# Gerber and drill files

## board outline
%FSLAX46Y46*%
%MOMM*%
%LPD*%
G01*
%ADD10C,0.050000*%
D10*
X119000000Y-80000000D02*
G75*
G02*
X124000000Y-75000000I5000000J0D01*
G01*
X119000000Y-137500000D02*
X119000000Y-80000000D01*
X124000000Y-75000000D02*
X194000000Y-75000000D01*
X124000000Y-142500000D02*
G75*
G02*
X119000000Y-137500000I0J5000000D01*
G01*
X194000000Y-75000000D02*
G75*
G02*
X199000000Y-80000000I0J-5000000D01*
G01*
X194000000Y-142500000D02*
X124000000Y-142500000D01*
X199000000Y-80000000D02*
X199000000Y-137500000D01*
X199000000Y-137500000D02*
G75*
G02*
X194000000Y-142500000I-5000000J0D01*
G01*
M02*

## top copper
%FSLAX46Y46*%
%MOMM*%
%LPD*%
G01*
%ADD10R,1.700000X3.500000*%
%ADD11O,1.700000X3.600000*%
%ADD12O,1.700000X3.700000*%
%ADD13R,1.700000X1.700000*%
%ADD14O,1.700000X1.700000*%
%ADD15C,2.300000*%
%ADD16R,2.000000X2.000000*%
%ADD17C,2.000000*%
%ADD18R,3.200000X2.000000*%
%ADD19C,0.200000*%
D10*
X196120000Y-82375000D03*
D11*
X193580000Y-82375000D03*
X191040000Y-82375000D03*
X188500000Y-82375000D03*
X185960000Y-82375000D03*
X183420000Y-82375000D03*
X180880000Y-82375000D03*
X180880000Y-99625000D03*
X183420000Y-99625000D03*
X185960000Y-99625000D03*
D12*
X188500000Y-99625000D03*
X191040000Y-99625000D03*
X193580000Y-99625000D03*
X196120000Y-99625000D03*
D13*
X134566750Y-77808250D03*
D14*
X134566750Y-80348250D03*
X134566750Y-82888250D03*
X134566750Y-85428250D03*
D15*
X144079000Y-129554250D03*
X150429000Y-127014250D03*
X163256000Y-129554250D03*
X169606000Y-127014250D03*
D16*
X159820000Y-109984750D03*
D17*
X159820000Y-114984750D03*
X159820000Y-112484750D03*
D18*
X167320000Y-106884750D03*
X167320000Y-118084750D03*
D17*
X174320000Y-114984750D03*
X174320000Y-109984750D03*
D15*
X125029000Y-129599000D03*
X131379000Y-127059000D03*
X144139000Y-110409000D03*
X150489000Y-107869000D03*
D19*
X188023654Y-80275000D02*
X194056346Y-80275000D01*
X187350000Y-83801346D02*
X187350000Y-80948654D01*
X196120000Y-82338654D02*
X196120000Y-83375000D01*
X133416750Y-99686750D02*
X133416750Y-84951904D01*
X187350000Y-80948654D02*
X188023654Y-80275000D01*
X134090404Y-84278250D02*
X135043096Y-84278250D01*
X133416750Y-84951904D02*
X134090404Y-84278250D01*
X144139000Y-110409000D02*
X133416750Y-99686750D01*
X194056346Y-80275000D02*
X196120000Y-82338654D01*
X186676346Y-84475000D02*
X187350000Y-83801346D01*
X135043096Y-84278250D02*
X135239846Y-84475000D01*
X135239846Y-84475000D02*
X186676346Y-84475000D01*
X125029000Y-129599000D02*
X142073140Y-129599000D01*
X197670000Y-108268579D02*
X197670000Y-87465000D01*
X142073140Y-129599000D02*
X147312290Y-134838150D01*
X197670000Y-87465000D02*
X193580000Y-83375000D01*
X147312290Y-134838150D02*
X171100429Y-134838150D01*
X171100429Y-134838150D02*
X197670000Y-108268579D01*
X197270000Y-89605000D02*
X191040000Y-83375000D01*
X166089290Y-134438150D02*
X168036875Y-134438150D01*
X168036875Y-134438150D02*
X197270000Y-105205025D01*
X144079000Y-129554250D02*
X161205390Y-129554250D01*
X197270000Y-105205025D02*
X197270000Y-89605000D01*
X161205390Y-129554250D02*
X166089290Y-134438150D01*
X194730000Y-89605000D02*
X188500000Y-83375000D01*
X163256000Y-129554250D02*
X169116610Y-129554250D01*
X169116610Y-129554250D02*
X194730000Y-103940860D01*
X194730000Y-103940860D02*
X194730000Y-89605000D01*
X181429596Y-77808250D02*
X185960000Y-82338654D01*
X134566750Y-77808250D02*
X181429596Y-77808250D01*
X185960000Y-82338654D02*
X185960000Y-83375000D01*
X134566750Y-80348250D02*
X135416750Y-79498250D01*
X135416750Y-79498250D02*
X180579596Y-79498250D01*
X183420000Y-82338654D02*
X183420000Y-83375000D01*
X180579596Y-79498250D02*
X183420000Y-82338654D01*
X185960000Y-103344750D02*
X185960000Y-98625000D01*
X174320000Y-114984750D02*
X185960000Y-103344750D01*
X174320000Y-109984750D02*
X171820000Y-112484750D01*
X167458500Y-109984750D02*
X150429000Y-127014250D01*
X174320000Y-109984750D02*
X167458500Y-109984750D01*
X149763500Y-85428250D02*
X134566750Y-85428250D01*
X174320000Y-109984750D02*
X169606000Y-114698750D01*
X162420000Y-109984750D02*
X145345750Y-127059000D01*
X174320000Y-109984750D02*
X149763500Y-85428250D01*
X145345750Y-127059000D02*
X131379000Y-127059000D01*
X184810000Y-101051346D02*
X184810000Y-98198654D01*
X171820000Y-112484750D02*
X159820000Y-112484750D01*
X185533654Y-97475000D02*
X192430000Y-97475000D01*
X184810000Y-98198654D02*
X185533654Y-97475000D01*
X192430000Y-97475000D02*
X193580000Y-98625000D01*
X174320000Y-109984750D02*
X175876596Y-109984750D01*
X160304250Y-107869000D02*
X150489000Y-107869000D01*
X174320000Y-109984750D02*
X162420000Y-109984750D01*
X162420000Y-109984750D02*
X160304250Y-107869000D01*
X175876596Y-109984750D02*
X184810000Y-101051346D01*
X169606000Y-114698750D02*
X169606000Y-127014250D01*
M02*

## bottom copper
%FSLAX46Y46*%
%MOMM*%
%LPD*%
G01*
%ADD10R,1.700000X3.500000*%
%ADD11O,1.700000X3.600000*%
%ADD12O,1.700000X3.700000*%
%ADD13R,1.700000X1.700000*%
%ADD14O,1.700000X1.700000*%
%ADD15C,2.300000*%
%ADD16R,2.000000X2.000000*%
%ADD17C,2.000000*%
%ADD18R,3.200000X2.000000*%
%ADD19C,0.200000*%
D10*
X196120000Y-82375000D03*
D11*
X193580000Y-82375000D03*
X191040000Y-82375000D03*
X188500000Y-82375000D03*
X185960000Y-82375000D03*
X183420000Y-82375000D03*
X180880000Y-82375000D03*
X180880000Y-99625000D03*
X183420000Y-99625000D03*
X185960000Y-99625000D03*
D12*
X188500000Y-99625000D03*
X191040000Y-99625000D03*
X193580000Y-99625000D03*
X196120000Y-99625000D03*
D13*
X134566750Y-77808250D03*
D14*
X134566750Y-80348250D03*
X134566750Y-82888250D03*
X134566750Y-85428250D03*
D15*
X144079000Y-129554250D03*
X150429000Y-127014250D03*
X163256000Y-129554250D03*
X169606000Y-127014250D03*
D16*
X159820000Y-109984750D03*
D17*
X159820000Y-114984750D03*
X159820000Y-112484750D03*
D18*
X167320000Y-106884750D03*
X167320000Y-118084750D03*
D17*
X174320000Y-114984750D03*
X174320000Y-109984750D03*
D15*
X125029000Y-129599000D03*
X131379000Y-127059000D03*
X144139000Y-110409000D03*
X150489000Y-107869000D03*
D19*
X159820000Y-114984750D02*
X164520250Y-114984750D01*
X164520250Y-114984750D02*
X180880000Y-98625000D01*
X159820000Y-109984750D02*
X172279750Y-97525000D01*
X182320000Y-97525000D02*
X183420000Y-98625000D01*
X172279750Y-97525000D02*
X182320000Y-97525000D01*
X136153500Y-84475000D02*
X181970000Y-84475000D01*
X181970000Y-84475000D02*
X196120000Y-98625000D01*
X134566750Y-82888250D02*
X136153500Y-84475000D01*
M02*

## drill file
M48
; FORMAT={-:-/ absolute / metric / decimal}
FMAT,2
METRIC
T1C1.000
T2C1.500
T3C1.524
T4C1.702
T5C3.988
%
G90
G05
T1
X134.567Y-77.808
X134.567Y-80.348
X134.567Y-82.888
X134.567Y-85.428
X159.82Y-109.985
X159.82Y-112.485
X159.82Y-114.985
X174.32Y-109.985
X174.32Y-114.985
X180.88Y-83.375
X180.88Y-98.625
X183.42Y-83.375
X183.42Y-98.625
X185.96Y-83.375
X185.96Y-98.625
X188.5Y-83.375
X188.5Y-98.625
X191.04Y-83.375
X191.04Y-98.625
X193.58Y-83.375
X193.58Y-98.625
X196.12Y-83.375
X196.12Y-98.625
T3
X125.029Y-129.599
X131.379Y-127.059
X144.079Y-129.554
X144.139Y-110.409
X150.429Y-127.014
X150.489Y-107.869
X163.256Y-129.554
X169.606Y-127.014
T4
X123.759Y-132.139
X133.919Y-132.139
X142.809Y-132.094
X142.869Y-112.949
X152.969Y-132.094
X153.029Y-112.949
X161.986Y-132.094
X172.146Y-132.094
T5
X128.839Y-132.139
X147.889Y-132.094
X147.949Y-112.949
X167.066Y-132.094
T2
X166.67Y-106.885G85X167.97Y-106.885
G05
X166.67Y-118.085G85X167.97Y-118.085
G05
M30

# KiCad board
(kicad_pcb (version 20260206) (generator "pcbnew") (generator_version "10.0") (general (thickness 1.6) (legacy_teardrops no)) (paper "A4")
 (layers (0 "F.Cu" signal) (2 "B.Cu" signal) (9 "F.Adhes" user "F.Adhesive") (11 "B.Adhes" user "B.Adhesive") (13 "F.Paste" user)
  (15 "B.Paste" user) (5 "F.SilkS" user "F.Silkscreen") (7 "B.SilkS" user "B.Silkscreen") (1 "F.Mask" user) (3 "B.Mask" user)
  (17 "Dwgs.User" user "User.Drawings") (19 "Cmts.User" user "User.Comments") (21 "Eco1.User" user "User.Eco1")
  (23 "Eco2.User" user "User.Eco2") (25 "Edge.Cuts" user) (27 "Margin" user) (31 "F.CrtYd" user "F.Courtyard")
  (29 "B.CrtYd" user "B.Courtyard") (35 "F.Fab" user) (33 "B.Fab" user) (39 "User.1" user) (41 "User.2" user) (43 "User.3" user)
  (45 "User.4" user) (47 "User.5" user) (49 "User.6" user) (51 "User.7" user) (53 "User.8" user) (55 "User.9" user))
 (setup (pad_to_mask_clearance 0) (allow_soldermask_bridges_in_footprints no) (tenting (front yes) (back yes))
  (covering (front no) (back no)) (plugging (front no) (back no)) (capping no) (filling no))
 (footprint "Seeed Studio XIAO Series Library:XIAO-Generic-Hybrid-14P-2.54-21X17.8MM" (layer "F.Cu") (at 188.5 91 -90)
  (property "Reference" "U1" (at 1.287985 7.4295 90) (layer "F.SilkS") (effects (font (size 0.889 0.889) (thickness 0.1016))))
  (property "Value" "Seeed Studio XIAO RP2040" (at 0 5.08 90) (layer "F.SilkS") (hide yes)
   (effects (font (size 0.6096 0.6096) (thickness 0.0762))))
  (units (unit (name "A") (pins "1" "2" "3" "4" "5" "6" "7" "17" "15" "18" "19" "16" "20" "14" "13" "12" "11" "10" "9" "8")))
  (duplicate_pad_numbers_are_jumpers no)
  (pad "1" thru_hole rect (at -7.625 -7.62 270) (size 3.5 1.7) (drill 1 (offset -1 0)) (layers "*.Cu" "*.Mask") (remove_unused_layers no)
   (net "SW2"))
  (pad "2" thru_hole oval (at -7.625 -5.08 270) (size 3.6 1.7) (drill 1 (offset -1 0)) (layers "*.Cu" "*.Mask") (remove_unused_layers no)
   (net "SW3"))
  (pad "3" thru_hole oval (at -7.625 -2.54 270) (size 3.6 1.7) (drill 1 (offset -1 0)) (layers "*.Cu" "*.Mask") (remove_unused_layers no)
   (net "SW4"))
  (pad "4" thru_hole oval (at -7.625 0 270) (size 3.6 1.7) (drill 1 (offset -1 0)) (layers "*.Cu" "*.Mask") (remove_unused_layers no)
   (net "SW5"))
  (pad "5" thru_hole oval (at -7.625 2.54 270) (size 3.6 1.7) (drill 1 (offset -1 0)) (layers "*.Cu" "*.Mask") (remove_unused_layers no)
   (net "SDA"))
  (pad "6" thru_hole oval (at -7.625 5.08 90) (size 3.6 1.7) (drill 1 (offset 1 0)) (layers "*.Cu" "*.Mask") (remove_unused_layers no)
   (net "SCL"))
  (pad "7" thru_hole oval (at -7.625 7.62 270) (size 3.6 1.7) (drill 1 (offset -1 0)) (layers "*.Cu" "*.Mask") (remove_unused_layers no)
   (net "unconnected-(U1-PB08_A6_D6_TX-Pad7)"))
  (pad "8" thru_hole oval (at 7.625 7.62 270) (size 3.6 1.7) (drill 1 (offset 1 0)) (layers "*.Cu" "*.Mask") (remove_unused_layers no)
   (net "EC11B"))
  (pad "9" thru_hole oval (at 7.625 5.08 270) (size 3.6 1.7) (drill 1 (offset 1 0)) (layers "*.Cu" "*.Mask") (remove_unused_layers no)
   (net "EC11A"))
  (pad "10" thru_hole oval (at 7.625 2.54 270) (size 3.6 1.7) (drill 1 (offset 1 0)) (layers "*.Cu" "*.Mask") (remove_unused_layers no)
   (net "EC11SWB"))
  (pad "11" thru_hole oval (at 7.625 0 270) (size 3.7 1.7) (drill 1 (offset 1 0)) (layers "*.Cu" "*.Mask") (remove_unused_layers no)
   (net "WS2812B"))
  (pad "12" thru_hole oval (at 7.625 -2.54 270) (size 3.7 1.7) (drill 1 (offset 1 0)) (layers "*.Cu" "*.Mask") (remove_unused_layers no)
   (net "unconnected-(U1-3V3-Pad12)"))
  (pad "13" thru_hole oval (at 7.625 -5.08 270) (size 3.7 1.7) (drill 1 (offset 1 0)) (layers "*.Cu" "*.Mask") (remove_unused_layers no)
   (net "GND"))
  (pad "14" thru_hole oval (at 7.625 -7.62 270) (size 3.7 1.7) (drill 1 (offset 1 0)) (layers "*.Cu" "*.Mask") (remove_unused_layers no)
   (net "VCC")))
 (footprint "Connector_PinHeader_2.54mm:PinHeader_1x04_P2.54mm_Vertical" (layer "F.Cu") (at 134.56675 77.80825)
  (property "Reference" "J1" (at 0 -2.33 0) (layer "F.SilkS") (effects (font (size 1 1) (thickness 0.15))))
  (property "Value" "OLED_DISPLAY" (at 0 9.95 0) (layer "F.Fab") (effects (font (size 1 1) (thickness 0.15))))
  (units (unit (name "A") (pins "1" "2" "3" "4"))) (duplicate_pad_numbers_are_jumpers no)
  (pad "1" thru_hole rect (at 0 0) (size 1.7 1.7) (drill 1) (layers "*.Cu" "*.Mask") (remove_unused_layers no) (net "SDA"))
  (pad "2" thru_hole oval (at 0 2.54) (size 1.7 1.7) (drill 1) (layers "*.Cu" "*.Mask") (remove_unused_layers no) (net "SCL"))
  (pad "3" thru_hole oval (at 0 5.08) (size 1.7 1.7) (drill 1) (layers "*.Cu" "*.Mask") (remove_unused_layers no) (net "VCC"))
  (pad "4" thru_hole oval (at 0 7.62) (size 1.7 1.7) (drill 1) (layers "*.Cu" "*.Mask") (remove_unused_layers no) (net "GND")))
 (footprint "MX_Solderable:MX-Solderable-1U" (layer "F.Cu") (at 147.889 132.09425)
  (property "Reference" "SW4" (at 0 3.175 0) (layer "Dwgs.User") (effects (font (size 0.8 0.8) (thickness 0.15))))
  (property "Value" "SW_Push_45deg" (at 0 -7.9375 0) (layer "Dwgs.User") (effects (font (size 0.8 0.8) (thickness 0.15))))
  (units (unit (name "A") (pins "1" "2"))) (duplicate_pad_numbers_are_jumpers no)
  (pad "" np_thru_hole circle (at -5.08 0 48.099) (size 1.7018 1.7018) (drill 1.7018) (layers "*.Cu" "*.Mask"))
  (pad "" np_thru_hole circle (at 0 0) (size 3.9878 3.9878) (drill 3.9878) (layers "*.Cu" "*.Mask"))
  (pad "" np_thru_hole circle (at 5.08 0 48.099) (size 1.7018 1.7018) (drill 1.7018) (layers "*.Cu" "*.Mask"))
  (pad "1" thru_hole circle (at -3.81 -2.54) (size 2.3 2.3) (drill 1.524) (layers "*.Cu" "B.Mask") (remove_unused_layers no) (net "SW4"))
  (pad "2" thru_hole circle (at 2.54 -5.08) (size 2.3 2.3) (drill 1.524) (layers "*.Cu" "B.Mask") (remove_unused_layers no) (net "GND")))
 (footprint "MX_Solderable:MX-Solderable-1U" (layer "F.Cu") (at 167.066 132.09425)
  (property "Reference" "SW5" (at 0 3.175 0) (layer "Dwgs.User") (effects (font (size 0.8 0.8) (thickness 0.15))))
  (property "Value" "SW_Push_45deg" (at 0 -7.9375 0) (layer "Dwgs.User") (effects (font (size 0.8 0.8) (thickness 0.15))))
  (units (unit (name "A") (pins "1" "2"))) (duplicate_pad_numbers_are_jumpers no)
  (pad "" np_thru_hole circle (at -5.08 0 48.099) (size 1.7018 1.7018) (drill 1.7018) (layers "*.Cu" "*.Mask"))
  (pad "" np_thru_hole circle (at 0 0) (size 3.9878 3.9878) (drill 3.9878) (layers "*.Cu" "*.Mask"))
  (pad "" np_thru_hole circle (at 5.08 0 48.099) (size 1.7018 1.7018) (drill 1.7018) (layers "*.Cu" "*.Mask"))
  (pad "1" thru_hole circle (at -3.81 -2.54) (size 2.3 2.3) (drill 1.524) (layers "*.Cu" "B.Mask") (remove_unused_layers no) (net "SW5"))
  (pad "2" thru_hole circle (at 2.54 -5.08) (size 2.3 2.3) (drill 1.524) (layers "*.Cu" "B.Mask") (remove_unused_layers no) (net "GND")))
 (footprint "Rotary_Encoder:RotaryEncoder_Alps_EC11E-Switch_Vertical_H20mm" (layer "F.Cu") (at 159.82 109.98475)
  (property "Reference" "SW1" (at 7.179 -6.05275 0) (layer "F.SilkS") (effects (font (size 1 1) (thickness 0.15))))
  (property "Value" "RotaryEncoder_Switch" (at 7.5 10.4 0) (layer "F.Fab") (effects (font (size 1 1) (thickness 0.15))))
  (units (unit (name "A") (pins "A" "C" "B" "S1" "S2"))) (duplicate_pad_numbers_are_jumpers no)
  (pad "A" thru_hole rect (at 0 0) (size 2 2) (drill 1) (layers "*.Cu" "*.Mask") (remove_unused_layers no) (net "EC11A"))
  (pad "B" thru_hole circle (at 0 5) (size 2 2) (drill 1) (layers "*.Cu" "*.Mask") (remove_unused_layers no) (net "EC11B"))
  (pad "C" thru_hole circle (at 0 2.5) (size 2 2) (drill 1) (layers "*.Cu" "*.Mask") (remove_unused_layers no) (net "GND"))
  (pad "MP" thru_hole rect (at 7.5 -3.1) (size 3.2 2) (drill oval 2.8 1.5) (layers "*.Cu" "*.Mask") (remove_unused_layers no))
  (pad "MP" thru_hole rect (at 7.5 8.1) (size 3.2 2) (drill oval 2.8 1.5) (layers "*.Cu" "*.Mask") (remove_unused_layers no))
  (pad "S1" thru_hole circle (at 14.5 5) (size 2 2) (drill 1) (layers "*.Cu" "*.Mask") (remove_unused_layers no) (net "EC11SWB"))
  (pad "S2" thru_hole circle (at 14.5 0) (size 2 2) (drill 1) (layers "*.Cu" "*.Mask") (remove_unused_layers no) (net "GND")))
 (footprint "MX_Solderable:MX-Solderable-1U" (layer "F.Cu") (at 128.839 132.139)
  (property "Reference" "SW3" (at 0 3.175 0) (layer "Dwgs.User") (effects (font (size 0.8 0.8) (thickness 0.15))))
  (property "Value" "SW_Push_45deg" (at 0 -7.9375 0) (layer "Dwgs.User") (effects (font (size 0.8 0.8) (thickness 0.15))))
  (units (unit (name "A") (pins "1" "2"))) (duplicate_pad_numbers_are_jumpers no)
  (pad "" np_thru_hole circle (at -5.08 0 48.099) (size 1.7018 1.7018) (drill 1.7018) (layers "*.Cu" "*.Mask"))
  (pad "" np_thru_hole circle (at 0 0) (size 3.9878 3.9878) (drill 3.9878) (layers "*.Cu" "*.Mask"))
  (pad "" np_thru_hole circle (at 5.08 0 48.099) (size 1.7018 1.7018) (drill 1.7018) (layers "*.Cu" "*.Mask"))
  (pad "1" thru_hole circle (at -3.81 -2.54) (size 2.3 2.3) (drill 1.524) (layers "*.Cu" "B.Mask") (remove_unused_layers no) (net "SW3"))
  (pad "2" thru_hole circle (at 2.54 -5.08) (size 2.3 2.3) (drill 1.524) (layers "*.Cu" "B.Mask") (remove_unused_layers no) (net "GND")))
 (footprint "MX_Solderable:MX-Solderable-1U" (layer "F.Cu") (at 147.949 112.949)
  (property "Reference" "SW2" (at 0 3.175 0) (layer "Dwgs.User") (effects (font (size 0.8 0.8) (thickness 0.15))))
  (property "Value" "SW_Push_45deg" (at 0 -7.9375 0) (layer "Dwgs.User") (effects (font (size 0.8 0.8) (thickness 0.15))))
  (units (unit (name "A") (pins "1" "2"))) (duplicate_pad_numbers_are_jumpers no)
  (pad "" np_thru_hole circle (at -5.08 0 48.099) (size 1.7018 1.7018) (drill 1.7018) (layers "*.Cu" "*.Mask"))
  (pad "" np_thru_hole circle (at 0 0) (size 3.9878 3.9878) (drill 3.9878) (layers "*.Cu" "*.Mask"))
  (pad "" np_thru_hole circle (at 5.08 0 48.099) (size 1.7018 1.7018) (drill 1.7018) (layers "*.Cu" "*.Mask"))
  (pad "1" thru_hole circle (at -3.81 -2.54) (size 2.3 2.3) (drill 1.524) (layers "*.Cu" "B.Mask") (remove_unused_layers no) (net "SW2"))
  (pad "2" thru_hole circle (at 2.54 -5.08) (size 2.3 2.3) (drill 1.524) (layers "*.Cu" "B.Mask") (remove_unused_layers no) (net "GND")))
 (gr_arc (start 119 80) (mid 120.464466 76.464466) (end 124 75) (stroke (width 0.05) (type default)) (layer "Edge.Cuts"))
 (gr_line (start 119 137.5) (end 119 80) (stroke (width 0.05) (type default)) (layer "Edge.Cuts"))
 (gr_line (start 124 75) (end 194 75) (stroke (width 0.05) (type default)) (layer "Edge.Cuts"))
 (gr_arc (start 124 142.5) (mid 120.464466 141.035534) (end 119 137.5) (stroke (width 0.05) (type default)) (layer "Edge.Cuts"))
 (gr_arc (start 194 75) (mid 197.535534 76.464466) (end 199 80) (stroke (width 0.05) (type default)) (layer "Edge.Cuts"))
 (gr_line (start 194 142.5) (end 124 142.5) (stroke (width 0.05) (type default)) (layer "Edge.Cuts"))
 (gr_line (start 199 80) (end 199 137.5) (stroke (width 0.05) (type default)) (layer "Edge.Cuts"))
 (gr_arc (start 199 137.5) (mid 197.535534 141.035534) (end 194 142.5) (stroke (width 0.05) (type default)) (layer "Edge.Cuts"))
 (segment (start 188.023654 80.275) (end 194.056346 80.275) (width 0.2) (layer "F.Cu") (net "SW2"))
 (segment (start 187.35 83.801346) (end 187.35 80.948654) (width 0.2) (layer "F.Cu") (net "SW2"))
 (segment (start 196.12 82.338654) (end 196.12 83.375) (width 0.2) (layer "F.Cu") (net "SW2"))
 (segment (start 133.41675 99.68675) (end 133.41675 84.951904) (width 0.2) (layer "F.Cu") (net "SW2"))
 (segment (start 187.35 80.948654) (end 188.023654 80.275) (width 0.2) (layer "F.Cu") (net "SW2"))
 (segment (start 134.090404 84.27825) (end 135.043096 84.27825) (width 0.2) (layer "F.Cu") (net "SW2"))
 (segment (start 133.41675 84.951904) (end 134.090404 84.27825) (width 0.2) (layer "F.Cu") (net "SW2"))
 (segment (start 144.139 110.409) (end 133.41675 99.68675) (width 0.2) (layer "F.Cu") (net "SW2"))
 (segment (start 194.056346 80.275) (end 196.12 82.338654) (width 0.2) (layer "F.Cu") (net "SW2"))
 (segment (start 186.676346 84.475) (end 187.35 83.801346) (width 0.2) (layer "F.Cu") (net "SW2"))
 (segment (start 135.043096 84.27825) (end 135.239846 84.475) (width 0.2) (layer "F.Cu") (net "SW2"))
 (segment (start 135.239846 84.475) (end 186.676346 84.475) (width 0.2) (layer "F.Cu") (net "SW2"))
 (segment (start 125.029 129.599) (end 142.07314 129.599) (width 0.2) (layer "F.Cu") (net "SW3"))
 (segment (start 197.67 108.268579) (end 197.67 87.465) (width 0.2) (layer "F.Cu") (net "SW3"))
 (segment (start 142.07314 129.599) (end 147.31229 134.83815) (width 0.2) (layer "F.Cu") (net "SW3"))
 (segment (start 197.67 87.465) (end 193.58 83.375) (width 0.2) (layer "F.Cu") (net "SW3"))
 (segment (start 147.31229 134.83815) (end 171.100429 134.83815) (width 0.2) (layer "F.Cu") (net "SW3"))
 (segment (start 171.100429 134.83815) (end 197.67 108.268579) (width 0.2) (layer "F.Cu") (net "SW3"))
 (segment (start 197.27 89.605) (end 191.04 83.375) (width 0.2) (layer "F.Cu") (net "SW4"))
 (segment (start 166.08929 134.43815) (end 168.036875 134.43815) (width 0.2) (layer "F.Cu") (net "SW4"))
 (segment (start 168.036875 134.43815) (end 197.27 105.205025) (width 0.2) (layer "F.Cu") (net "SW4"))
 (segment (start 144.079 129.55425) (end 161.20539 129.55425) (width 0.2) (layer "F.Cu") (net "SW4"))
 (segment (start 197.27 105.205025) (end 197.27 89.605) (width 0.2) (layer "F.Cu") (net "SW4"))
 (segment (start 161.20539 129.55425) (end 166.08929 134.43815) (width 0.2) (layer "F.Cu") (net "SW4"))
 (segment (start 194.73 89.605) (end 188.5 83.375) (width 0.2) (layer "F.Cu") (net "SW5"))
 (segment (start 163.256 129.55425) (end 169.11661 129.55425) (width 0.2) (layer "F.Cu") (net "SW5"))
 (segment (start 169.11661 129.55425) (end 194.73 103.94086) (width 0.2) (layer "F.Cu") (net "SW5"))
 (segment (start 194.73 103.94086) (end 194.73 89.605) (width 0.2) (layer "F.Cu") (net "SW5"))
 (segment (start 181.429596 77.80825) (end 185.96 82.338654) (width 0.2) (layer "F.Cu") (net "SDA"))
 (segment (start 134.56675 77.80825) (end 181.429596 77.80825) (width 0.2) (layer "F.Cu") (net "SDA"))
 (segment (start 185.96 82.338654) (end 185.96 83.375) (width 0.2) (layer "F.Cu") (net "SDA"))
 (segment (start 134.56675 80.34825) (end 135.41675 79.49825) (width 0.2) (layer "F.Cu") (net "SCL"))
 (segment (start 135.41675 79.49825) (end 180.579596 79.49825) (width 0.2) (layer "F.Cu") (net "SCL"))
 (segment (start 183.42 82.338654) (end 183.42 83.375) (width 0.2) (layer "F.Cu") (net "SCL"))
 (segment (start 180.579596 79.49825) (end 183.42 82.338654) (width 0.2) (layer "F.Cu") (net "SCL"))
 (segment (start 159.82 114.98475) (end 164.52025 114.98475) (width 0.2) (layer "B.Cu") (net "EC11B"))
 (segment (start 164.52025 114.98475) (end 180.88 98.625) (width 0.2) (layer "B.Cu") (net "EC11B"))
 (segment (start 159.82 109.98475) (end 172.27975 97.525) (width 0.2) (layer "B.Cu") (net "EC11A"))
 (segment (start 182.32 97.525) (end 183.42 98.625) (width 0.2) (layer "B.Cu") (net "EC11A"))
 (segment (start 172.27975 97.525) (end 182.32 97.525) (width 0.2) (layer "B.Cu") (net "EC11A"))
 (segment (start 185.96 103.34475) (end 185.96 98.625) (width 0.2) (layer "F.Cu") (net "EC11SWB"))
 (segment (start 174.32 114.98475) (end 185.96 103.34475) (width 0.2) (layer "F.Cu") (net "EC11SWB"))
 (segment (start 174.32 109.98475) (end 171.82 112.48475) (width 0.2) (layer "F.Cu") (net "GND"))
 (segment (start 167.4585 109.98475) (end 150.429 127.01425) (width 0.2) (layer "F.Cu") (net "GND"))
 (segment (start 174.32 109.98475) (end 167.4585 109.98475) (width 0.2) (layer "F.Cu") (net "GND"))
 (segment (start 149.7635 85.42825) (end 134.56675 85.42825) (width 0.2) (layer "F.Cu") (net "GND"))
 (segment (start 174.32 109.98475) (end 169.606 114.69875) (width 0.2) (layer "F.Cu") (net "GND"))
 (segment (start 162.42 109.98475) (end 145.34575 127.059) (width 0.2) (layer "F.Cu") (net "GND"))
 (segment (start 174.32 109.98475) (end 149.7635 85.42825) (width 0.2) (layer "F.Cu") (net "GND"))
 (segment (start 145.34575 127.059) (end 131.379 127.059) (width 0.2) (layer "F.Cu") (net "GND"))
 (segment (start 184.81 101.051346) (end 184.81 98.198654) (width 0.2) (layer "F.Cu") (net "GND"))
 (segment (start 171.82 112.48475) (end 159.82 112.48475) (width 0.2) (layer "F.Cu") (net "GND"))
 (segment (start 185.533654 97.475) (end 192.43 97.475) (width 0.2) (layer "F.Cu") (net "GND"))
 (segment (start 184.81 98.198654) (end 185.533654 97.475) (width 0.2) (layer "F.Cu") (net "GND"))
 (segment (start 192.43 97.475) (end 193.58 98.625) (width 0.2) (layer "F.Cu") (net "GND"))
 (segment (start 174.32 109.98475) (end 175.876596 109.98475) (width 0.2) (layer "F.Cu") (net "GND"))
 (segment (start 160.30425 107.869) (end 150.489 107.869) (width 0.2) (layer "F.Cu") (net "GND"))
 (segment (start 174.32 109.98475) (end 162.42 109.98475) (width 0.2) (layer "F.Cu") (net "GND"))
 (segment (start 162.42 109.98475) (end 160.30425 107.869) (width 0.2) (layer "F.Cu") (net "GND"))
 (segment (start 175.876596 109.98475) (end 184.81 101.051346) (width 0.2) (layer "F.Cu") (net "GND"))
 (segment (start 169.606 114.69875) (end 169.606 127.01425) (width 0.2) (layer "F.Cu") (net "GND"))
 (segment (start 136.1535 84.475) (end 181.97 84.475) (width 0.2) (layer "B.Cu") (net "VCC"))
 (segment (start 181.97 84.475) (end 196.12 98.625) (width 0.2) (layer "B.Cu") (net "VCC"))
 (segment (start 134.56675 82.88825) (end 136.1535 84.475) (width 0.2) (layer "B.Cu") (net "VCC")))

